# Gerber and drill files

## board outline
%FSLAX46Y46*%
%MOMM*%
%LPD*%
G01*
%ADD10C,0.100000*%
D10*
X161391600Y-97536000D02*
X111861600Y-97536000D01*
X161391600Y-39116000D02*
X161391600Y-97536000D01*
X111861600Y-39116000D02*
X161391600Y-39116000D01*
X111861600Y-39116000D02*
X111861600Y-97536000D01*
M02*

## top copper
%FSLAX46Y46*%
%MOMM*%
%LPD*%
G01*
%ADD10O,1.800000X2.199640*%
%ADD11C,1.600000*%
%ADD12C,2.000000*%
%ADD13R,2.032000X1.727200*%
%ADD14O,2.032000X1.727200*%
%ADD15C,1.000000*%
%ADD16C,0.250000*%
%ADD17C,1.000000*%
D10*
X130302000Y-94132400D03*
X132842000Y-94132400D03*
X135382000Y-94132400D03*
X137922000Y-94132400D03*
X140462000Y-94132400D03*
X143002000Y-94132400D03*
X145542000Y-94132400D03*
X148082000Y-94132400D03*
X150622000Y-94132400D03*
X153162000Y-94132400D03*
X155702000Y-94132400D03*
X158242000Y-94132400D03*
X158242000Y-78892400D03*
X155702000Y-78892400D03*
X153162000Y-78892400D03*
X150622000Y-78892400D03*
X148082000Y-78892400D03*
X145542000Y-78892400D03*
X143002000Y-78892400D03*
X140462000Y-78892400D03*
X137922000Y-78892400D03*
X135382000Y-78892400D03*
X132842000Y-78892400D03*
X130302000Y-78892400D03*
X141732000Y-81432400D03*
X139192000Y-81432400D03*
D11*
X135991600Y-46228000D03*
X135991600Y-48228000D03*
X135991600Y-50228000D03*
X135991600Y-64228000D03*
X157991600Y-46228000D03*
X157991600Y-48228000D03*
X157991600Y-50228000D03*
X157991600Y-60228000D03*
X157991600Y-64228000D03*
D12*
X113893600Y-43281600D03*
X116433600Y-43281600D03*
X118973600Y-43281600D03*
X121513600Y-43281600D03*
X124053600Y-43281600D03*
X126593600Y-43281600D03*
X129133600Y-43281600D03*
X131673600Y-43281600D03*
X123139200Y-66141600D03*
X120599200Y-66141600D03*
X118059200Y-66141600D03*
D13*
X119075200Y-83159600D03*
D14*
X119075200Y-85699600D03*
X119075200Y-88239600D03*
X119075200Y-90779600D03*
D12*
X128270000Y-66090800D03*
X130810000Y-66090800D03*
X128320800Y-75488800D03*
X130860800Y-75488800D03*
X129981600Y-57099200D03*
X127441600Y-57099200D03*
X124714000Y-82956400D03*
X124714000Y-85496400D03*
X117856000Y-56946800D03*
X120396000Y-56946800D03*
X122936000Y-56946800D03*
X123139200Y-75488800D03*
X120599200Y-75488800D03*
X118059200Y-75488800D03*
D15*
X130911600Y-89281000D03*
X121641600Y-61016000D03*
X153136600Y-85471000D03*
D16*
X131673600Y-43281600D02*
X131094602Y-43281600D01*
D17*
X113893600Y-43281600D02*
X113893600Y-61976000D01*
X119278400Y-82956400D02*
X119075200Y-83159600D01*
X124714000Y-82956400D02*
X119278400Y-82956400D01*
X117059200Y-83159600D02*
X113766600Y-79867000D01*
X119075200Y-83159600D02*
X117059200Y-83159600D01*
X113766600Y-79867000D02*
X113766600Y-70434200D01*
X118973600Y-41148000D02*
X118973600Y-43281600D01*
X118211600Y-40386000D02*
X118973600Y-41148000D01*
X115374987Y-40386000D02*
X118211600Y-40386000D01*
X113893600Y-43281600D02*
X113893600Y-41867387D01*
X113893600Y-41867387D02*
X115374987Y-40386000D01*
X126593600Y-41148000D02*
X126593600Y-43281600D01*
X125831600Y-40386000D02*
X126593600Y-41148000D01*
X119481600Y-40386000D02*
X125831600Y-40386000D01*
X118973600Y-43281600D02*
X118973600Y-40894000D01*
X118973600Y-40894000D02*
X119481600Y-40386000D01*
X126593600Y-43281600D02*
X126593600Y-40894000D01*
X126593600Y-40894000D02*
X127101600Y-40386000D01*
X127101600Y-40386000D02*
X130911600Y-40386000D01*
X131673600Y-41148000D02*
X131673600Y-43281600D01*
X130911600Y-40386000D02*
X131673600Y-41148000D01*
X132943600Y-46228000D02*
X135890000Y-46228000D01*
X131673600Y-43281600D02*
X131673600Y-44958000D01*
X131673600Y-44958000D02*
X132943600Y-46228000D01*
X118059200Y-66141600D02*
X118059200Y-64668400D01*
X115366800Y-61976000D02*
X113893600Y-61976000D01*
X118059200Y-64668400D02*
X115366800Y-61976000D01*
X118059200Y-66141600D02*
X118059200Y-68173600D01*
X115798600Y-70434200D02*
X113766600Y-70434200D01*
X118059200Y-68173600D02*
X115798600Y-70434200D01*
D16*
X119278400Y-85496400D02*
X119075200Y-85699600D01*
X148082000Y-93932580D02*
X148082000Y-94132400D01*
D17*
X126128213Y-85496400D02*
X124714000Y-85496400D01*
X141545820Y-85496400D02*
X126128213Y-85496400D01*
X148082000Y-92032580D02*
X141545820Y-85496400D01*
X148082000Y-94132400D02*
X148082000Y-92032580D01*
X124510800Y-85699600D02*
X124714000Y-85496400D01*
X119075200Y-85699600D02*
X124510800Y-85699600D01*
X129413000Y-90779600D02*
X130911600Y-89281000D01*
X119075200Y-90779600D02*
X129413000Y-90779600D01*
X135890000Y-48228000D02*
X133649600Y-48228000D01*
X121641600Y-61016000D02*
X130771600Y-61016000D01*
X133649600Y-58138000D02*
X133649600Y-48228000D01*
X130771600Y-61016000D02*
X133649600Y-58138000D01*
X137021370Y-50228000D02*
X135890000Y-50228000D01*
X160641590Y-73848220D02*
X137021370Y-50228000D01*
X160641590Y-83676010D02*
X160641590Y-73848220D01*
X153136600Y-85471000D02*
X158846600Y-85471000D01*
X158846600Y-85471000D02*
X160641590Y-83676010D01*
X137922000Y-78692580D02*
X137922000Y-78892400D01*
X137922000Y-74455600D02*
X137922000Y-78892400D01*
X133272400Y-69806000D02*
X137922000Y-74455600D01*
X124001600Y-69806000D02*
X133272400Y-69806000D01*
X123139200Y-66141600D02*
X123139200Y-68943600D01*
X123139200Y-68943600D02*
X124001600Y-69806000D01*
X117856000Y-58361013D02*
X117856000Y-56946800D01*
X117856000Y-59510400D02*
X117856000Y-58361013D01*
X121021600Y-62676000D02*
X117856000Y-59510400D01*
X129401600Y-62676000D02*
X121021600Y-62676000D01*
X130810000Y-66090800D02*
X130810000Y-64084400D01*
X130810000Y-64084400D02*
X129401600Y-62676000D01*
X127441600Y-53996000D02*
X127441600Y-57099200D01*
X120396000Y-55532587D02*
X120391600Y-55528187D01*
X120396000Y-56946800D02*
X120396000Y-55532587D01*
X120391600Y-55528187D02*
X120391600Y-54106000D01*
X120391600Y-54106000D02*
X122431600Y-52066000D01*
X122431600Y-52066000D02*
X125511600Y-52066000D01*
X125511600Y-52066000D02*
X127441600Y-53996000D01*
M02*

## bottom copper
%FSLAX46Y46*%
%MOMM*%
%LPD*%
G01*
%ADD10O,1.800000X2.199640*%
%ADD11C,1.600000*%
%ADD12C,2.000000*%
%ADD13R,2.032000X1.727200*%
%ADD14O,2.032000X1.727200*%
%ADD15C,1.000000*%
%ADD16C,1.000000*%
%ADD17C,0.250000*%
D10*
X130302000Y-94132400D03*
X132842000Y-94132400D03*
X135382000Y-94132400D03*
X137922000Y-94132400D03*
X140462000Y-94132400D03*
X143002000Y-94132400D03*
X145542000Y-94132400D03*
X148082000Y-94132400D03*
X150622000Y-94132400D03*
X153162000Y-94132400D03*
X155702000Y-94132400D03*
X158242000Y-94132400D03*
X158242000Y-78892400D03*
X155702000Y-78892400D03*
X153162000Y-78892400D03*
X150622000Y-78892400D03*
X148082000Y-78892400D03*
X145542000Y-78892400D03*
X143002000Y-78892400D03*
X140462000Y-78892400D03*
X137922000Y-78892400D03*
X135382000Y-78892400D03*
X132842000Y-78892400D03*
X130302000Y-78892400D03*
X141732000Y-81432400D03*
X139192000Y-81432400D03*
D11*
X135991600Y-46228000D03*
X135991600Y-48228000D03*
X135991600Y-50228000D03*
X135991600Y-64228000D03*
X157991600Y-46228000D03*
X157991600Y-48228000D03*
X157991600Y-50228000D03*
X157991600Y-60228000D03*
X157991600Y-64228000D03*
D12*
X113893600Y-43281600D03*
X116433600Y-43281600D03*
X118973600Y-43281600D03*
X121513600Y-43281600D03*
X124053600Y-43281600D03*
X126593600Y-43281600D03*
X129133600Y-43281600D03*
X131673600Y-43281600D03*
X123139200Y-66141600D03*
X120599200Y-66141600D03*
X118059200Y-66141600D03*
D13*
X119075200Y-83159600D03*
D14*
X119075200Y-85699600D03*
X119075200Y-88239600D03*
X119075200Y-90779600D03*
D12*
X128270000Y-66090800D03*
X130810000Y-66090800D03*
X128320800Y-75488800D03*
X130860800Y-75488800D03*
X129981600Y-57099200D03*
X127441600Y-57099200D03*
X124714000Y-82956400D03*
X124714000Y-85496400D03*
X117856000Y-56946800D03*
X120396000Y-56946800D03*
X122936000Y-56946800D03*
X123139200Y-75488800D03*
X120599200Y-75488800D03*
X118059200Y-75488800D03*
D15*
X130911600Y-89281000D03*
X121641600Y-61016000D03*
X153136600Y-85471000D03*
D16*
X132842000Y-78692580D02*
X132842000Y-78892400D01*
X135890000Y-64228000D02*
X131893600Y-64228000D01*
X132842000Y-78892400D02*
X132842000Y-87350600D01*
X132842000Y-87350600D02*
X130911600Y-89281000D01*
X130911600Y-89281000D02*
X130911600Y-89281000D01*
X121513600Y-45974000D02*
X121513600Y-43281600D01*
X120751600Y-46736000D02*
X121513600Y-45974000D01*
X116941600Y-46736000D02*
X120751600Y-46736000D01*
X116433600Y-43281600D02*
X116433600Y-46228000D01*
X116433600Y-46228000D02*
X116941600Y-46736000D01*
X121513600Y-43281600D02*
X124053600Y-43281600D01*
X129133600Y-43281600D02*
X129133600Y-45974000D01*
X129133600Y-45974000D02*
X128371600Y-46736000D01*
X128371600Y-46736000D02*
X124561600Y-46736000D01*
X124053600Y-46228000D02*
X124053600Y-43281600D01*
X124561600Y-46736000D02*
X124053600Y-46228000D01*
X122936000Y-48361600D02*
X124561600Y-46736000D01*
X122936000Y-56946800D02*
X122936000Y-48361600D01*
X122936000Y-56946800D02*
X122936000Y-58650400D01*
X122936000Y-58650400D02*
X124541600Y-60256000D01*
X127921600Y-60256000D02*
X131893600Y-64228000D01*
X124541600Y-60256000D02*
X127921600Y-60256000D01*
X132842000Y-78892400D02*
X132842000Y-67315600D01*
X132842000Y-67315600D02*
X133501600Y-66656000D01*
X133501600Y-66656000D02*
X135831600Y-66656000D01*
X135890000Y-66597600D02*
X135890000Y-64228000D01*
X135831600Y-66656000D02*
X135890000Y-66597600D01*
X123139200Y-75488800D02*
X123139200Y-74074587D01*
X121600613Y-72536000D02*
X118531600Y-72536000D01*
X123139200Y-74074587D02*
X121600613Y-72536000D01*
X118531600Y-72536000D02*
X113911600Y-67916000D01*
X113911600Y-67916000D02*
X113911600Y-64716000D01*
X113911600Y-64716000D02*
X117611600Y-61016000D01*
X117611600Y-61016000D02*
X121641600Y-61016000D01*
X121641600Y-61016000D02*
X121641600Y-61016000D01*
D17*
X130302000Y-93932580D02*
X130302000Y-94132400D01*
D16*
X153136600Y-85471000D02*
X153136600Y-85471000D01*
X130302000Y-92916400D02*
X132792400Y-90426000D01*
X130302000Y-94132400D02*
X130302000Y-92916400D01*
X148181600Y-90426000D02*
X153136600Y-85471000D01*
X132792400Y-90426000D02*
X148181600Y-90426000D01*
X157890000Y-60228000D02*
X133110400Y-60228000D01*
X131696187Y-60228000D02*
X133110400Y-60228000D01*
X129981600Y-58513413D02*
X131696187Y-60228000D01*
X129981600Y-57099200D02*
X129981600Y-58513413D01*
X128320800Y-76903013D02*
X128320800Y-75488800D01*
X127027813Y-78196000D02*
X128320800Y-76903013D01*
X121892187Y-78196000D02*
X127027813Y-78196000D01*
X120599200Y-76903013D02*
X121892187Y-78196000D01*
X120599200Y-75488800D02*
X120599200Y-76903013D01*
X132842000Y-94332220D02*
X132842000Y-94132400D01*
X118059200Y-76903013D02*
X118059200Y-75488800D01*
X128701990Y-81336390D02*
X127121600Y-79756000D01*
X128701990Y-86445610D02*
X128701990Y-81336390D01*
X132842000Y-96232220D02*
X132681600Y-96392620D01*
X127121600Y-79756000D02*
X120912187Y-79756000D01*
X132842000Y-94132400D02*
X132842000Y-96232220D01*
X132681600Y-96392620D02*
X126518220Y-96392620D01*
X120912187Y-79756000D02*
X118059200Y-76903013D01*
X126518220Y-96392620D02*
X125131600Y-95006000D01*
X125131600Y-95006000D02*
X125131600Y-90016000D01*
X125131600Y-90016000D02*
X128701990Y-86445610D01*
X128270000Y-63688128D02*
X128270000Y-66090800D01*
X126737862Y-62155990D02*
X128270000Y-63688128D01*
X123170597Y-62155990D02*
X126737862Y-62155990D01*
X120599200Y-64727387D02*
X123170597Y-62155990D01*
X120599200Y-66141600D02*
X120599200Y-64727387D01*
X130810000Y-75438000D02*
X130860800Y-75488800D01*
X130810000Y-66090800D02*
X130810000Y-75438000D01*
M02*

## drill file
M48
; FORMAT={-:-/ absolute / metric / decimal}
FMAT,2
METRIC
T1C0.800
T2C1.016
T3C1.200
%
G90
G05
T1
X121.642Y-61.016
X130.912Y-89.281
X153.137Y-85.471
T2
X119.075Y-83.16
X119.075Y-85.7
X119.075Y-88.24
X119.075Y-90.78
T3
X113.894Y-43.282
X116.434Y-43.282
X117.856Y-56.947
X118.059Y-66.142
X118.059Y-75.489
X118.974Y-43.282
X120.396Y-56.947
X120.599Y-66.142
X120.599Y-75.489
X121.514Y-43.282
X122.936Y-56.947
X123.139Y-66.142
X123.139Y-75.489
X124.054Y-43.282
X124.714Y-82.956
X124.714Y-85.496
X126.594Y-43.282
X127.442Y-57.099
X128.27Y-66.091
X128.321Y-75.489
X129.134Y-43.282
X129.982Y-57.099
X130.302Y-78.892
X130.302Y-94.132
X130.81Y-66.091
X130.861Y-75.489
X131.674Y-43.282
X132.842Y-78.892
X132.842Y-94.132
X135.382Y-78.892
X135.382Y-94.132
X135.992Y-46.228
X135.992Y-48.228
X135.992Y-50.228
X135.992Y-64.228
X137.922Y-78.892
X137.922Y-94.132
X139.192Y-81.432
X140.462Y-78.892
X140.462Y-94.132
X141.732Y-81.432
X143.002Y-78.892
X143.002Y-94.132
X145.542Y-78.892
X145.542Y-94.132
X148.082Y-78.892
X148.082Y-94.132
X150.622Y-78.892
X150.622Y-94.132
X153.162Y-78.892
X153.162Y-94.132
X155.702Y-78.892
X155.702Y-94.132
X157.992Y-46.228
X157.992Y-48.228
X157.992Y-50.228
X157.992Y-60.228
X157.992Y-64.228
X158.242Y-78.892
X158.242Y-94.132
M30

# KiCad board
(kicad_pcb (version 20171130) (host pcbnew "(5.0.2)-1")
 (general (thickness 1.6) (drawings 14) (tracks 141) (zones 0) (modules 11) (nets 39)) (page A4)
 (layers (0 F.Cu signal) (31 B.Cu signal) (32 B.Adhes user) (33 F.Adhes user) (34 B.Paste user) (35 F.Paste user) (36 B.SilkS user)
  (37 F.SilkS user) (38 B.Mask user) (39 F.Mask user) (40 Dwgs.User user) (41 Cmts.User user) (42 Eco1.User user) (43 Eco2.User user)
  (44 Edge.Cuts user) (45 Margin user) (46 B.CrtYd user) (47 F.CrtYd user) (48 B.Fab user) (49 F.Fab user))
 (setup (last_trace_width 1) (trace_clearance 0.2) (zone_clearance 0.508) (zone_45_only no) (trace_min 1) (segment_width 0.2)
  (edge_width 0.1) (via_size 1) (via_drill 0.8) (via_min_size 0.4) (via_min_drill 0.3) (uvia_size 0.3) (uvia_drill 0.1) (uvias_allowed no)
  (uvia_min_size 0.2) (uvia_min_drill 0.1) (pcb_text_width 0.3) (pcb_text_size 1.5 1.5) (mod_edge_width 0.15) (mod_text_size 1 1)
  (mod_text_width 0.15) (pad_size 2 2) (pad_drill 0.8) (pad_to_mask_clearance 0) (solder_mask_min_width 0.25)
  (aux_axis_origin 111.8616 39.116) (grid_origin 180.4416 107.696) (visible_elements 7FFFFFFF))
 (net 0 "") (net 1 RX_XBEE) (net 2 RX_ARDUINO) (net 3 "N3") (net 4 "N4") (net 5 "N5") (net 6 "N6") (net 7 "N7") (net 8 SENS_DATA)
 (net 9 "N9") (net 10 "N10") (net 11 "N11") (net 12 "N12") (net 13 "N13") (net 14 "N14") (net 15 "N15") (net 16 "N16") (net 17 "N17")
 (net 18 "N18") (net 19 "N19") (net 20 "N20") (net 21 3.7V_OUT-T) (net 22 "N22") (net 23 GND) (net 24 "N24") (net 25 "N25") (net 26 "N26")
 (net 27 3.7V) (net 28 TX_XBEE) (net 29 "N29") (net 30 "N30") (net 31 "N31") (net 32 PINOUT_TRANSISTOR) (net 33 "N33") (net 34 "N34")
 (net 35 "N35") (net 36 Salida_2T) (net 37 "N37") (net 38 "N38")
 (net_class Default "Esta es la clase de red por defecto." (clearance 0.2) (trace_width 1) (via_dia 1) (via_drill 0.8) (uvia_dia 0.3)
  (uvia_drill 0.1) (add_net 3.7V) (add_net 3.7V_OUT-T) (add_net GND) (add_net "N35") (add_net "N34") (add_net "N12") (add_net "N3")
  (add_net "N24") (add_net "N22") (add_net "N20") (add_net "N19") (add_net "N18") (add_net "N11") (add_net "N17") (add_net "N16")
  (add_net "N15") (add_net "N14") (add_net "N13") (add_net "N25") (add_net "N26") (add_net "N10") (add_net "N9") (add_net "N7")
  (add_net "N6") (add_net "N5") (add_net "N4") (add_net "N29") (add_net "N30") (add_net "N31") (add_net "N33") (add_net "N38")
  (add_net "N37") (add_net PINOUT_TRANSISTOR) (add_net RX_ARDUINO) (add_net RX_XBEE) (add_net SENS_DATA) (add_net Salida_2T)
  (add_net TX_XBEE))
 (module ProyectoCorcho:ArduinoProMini (layer F.Cu) (at 144.272 86.5124)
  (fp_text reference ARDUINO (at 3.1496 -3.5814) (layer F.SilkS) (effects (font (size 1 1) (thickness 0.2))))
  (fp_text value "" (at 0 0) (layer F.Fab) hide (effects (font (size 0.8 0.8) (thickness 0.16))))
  (pad 12 thru_hole oval (at -13.97 7.62) (size 1.8 2.19964) (drill 1.2) (layers *.Cu *.Mask) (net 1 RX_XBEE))
  (pad 11 thru_hole oval (at -11.43 7.62) (size 1.8 2.19964) (drill 1.2) (layers *.Cu *.Mask) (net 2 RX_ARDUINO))
  (pad 10 thru_hole oval (at -8.89 7.62) (size 1.8 2.19964) (drill 1.2) (layers *.Cu *.Mask) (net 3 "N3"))
  (pad 9 thru_hole oval (at -6.35 7.62) (size 1.8 2.19964) (drill 1.2) (layers *.Cu *.Mask) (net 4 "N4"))
  (pad 8 thru_hole oval (at -3.81 7.62) (size 1.8 2.19964) (drill 1.2) (layers *.Cu *.Mask) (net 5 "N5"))
  (pad 7 thru_hole oval (at -1.27 7.62) (size 1.8 2.19964) (drill 1.2) (layers *.Cu *.Mask) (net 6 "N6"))
  (pad 6 thru_hole oval (at 1.27 7.62) (size 1.8 2.19964) (drill 1.2) (layers *.Cu *.Mask) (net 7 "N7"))
  (pad 5 thru_hole oval (at 3.81 7.62) (size 1.8 2.19964) (drill 1.2) (layers *.Cu *.Mask) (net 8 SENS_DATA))
  (pad 4 thru_hole oval (at 6.35 7.62) (size 1.8 2.19964) (drill 1.2) (layers *.Cu *.Mask) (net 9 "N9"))
  (pad 3 thru_hole oval (at 8.89 7.62) (size 1.8 2.19964) (drill 1.2) (layers *.Cu *.Mask) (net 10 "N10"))
  (pad 2 thru_hole oval (at 11.43 7.62) (size 1.8 2.19964) (drill 1.2) (layers *.Cu *.Mask) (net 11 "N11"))
  (pad 1 thru_hole oval (at 13.97 7.62) (size 1.8 2.19964) (drill 1.2) (layers *.Cu *.Mask) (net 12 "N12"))
  (pad 24 thru_hole oval (at 13.97 -7.62) (size 1.8 2.19964) (drill 1.2) (layers *.Cu *.Mask) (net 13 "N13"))
  (pad 23 thru_hole oval (at 11.43 -7.62) (size 1.8 2.19964) (drill 1.2) (layers *.Cu *.Mask) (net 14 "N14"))
  (pad 22 thru_hole oval (at 8.89 -7.62) (size 1.8 2.19964) (drill 1.2) (layers *.Cu *.Mask) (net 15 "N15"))
  (pad 21 thru_hole oval (at 6.35 -7.62) (size 1.8 2.19964) (drill 1.2) (layers *.Cu *.Mask) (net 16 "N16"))
  (pad 20 thru_hole oval (at 3.81 -7.62) (size 1.8 2.19964) (drill 1.2) (layers *.Cu *.Mask) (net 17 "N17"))
  (pad 19 thru_hole oval (at 1.27 -7.62) (size 1.8 2.19964) (drill 1.2) (layers *.Cu *.Mask) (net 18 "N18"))
  (pad 18 thru_hole oval (at -1.27 -7.62) (size 1.8 2.19964) (drill 1.2) (layers *.Cu *.Mask) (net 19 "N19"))
  (pad 17 thru_hole oval (at -3.81 -7.62) (size 1.8 2.19964) (drill 1.2) (layers *.Cu *.Mask) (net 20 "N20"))
  (pad 16 thru_hole oval (at -6.35 -7.62) (size 1.8 2.19964) (drill 1.2) (layers *.Cu *.Mask) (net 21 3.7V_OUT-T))
  (pad 15 thru_hole oval (at -8.89 -7.62) (size 1.8 2.19964) (drill 1.2) (layers *.Cu *.Mask) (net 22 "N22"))
  (pad 14 thru_hole oval (at -11.43 -7.62) (size 1.8 2.19964) (drill 1.2) (layers *.Cu *.Mask) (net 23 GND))
  (pad 13 thru_hole oval (at -13.97 -7.62) (size 1.8 2.19964) (drill 1.2) (layers *.Cu *.Mask) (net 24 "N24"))
  (pad 25 thru_hole oval (at -2.54 -5.08) (size 1.8 2.19964) (drill 1.2) (layers *.Cu *.Mask) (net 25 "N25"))
  (pad 26 thru_hole oval (at -5.08 -5.08) (size 1.8 2.19964) (drill 1.2) (layers *.Cu *.Mask) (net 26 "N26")))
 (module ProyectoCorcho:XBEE (layer F.Cu) (at 134.7216 44.958)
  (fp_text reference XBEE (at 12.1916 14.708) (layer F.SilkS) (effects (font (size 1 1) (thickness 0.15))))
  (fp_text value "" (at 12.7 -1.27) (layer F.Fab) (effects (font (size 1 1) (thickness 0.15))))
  (pad 1 thru_hole circle (at 1.27 1.27) (size 1.6 1.6) (drill 1.2) (layers *.Cu *.Mask) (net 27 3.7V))
  (pad 2 thru_hole circle (at 1.27 3.27) (size 1.6 1.6) (drill 1.2) (layers *.Cu *.Mask) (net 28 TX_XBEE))
  (pad 3 thru_hole circle (at 1.27 5.27) (size 1.6 1.6) (drill 1.2) (layers *.Cu *.Mask) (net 1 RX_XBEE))
  (pad 4 thru_hole circle (at 1.27 19.27) (size 1.6 1.6) (drill 1.2) (layers *.Cu *.Mask) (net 23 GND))
  (pad 5 thru_hole circle (at 23.27 1.27) (size 1.6 1.6) (drill 1.2) (layers *.Cu *.Mask) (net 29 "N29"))
  (pad 6 thru_hole circle (at 23.27 3.27) (size 1.6 1.6) (drill 1.2) (layers *.Cu *.Mask) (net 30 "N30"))
  (pad 7 thru_hole circle (at 23.27 5.27) (size 1.6 1.6) (drill 1.2) (layers *.Cu *.Mask) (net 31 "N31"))
  (pad 8 thru_hole circle (at 23.27 15.27) (size 1.6 1.6) (drill 1.2) (layers *.Cu *.Mask) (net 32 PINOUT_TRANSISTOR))
  (pad 9 thru_hole circle (at 23.27 19.27) (size 1.6 1.6) (drill 1.2) (layers *.Cu *.Mask) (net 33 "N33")))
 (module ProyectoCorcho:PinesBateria (layer F.Cu) (at 112.6236 42.0116)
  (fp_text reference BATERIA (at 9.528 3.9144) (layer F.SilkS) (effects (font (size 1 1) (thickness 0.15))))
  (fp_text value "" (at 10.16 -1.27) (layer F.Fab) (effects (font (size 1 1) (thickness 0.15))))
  (pad 1 thru_hole circle (at 1.27 1.27) (size 2 2) (drill 1.2) (layers *.Cu *.Mask) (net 27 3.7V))
  (pad 2 thru_hole circle (at 3.81 1.27) (size 2 2) (drill 1.2) (layers *.Cu *.Mask) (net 23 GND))
  (pad 3 thru_hole circle (at 6.35 1.27) (size 2 2) (drill 1.2) (layers *.Cu *.Mask) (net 27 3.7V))
  (pad 4 thru_hole circle (at 8.89 1.27) (size 2 2) (drill 1.2) (layers *.Cu *.Mask) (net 23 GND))
  (pad 5 thru_hole circle (at 11.43 1.27) (size 2 2) (drill 1.2) (layers *.Cu *.Mask) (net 23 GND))
  (pad 6 thru_hole circle (at 13.97 1.27) (size 2 2) (drill 1.2) (layers *.Cu *.Mask) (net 27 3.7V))
  (pad 7 thru_hole circle (at 16.51 1.27) (size 2 2) (drill 1.2) (layers *.Cu *.Mask) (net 23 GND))
  (pad 8 thru_hole circle (at 19.05 1.27) (size 2 2) (drill 1.2) (layers *.Cu *.Mask) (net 27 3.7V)))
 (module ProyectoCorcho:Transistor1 (layer B.Cu) (at 120.5992 66.1416)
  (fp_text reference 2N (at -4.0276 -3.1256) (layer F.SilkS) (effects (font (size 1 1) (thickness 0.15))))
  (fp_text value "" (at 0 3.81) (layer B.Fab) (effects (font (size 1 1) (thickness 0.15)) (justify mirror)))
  (pad 3 thru_hole circle (at 2.54 0) (size 2 2) (drill 1.2) (layers *.Cu *.Mask) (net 21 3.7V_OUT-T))
  (pad 2 thru_hole circle (at 0 0) (size 2 2) (drill 1.2) (layers *.Cu *.Mask) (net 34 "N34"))
  (pad 1 thru_hole circle (at -2.54 0) (size 2 2) (drill 1.2) (layers *.Cu *.Mask) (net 27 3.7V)))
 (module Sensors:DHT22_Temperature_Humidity (layer F.Cu) (at 119.0752 86.9696 270)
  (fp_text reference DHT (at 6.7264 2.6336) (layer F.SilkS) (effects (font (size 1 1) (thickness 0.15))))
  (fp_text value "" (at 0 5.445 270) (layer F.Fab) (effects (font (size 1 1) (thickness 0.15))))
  (pad 1 thru_hole rect (at -3.81 0) (size 2.032 1.7272) (drill 1.016) (layers *.Cu *.Mask F.SilkS) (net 27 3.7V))
  (pad 2 thru_hole oval (at -1.27 0) (size 2.032 1.7272) (drill 1.016) (layers *.Cu *.Mask F.SilkS) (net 8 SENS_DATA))
  (pad 3 thru_hole oval (at 1.27 0) (size 2.032 1.7272) (drill 1.016) (layers *.Cu *.Mask F.SilkS) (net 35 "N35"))
  (pad 4 thru_hole oval (at 3.81 0) (size 2.032 1.7272) (drill 1.016) (layers *.Cu *.Mask F.SilkS) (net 23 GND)))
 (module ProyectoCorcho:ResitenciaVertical (layer F.Cu) (at 128.27 66.0908)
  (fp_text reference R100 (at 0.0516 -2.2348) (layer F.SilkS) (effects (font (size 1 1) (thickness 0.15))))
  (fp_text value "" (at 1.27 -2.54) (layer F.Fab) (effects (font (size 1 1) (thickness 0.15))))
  (pad 1 thru_hole circle (at 0 0) (size 2 2) (drill 1.2) (layers *.Cu *.Mask) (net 34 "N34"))
  (pad 2 thru_hole circle (at 2.54 0) (size 2 2) (drill 1.2) (layers *.Cu *.Mask) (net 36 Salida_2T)))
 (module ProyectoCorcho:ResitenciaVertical (layer F.Cu) (at 128.3208 75.4888)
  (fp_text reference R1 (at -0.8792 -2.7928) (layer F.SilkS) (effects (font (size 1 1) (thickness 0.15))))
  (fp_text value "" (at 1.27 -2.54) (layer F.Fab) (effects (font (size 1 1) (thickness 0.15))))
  (pad 1 thru_hole circle (at 0 0) (size 2 2) (drill 1.2) (layers *.Cu *.Mask) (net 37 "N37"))
  (pad 2 thru_hole circle (at 2.54 0) (size 2 2) (drill 1.2) (layers *.Cu *.Mask) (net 36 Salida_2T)))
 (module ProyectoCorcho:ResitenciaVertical (layer F.Cu) (at 127.4416 57.0992)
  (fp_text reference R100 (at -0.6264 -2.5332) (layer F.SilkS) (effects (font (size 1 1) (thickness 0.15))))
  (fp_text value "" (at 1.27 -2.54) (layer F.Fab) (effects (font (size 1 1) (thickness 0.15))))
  (pad 2 thru_hole circle (at 2.54 0) (size 2 2) (drill 1.2) (layers *.Cu *.Mask) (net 32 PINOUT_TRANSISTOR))
  (pad 1 thru_hole circle (at 0 0) (size 2 2) (drill 1.2) (layers *.Cu *.Mask) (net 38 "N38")))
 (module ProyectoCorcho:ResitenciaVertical (layer F.Cu) (at 124.714 82.9564 270)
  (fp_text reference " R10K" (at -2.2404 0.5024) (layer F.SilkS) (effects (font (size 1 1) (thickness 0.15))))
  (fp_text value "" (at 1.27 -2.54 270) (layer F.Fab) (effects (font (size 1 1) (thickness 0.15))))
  (pad 1 thru_hole circle (at 0 0 270) (size 2 2) (drill 1.2) (layers *.Cu *.Mask) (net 27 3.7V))
  (pad 2 thru_hole circle (at 2.54 0 270) (size 2 2) (drill 1.2) (layers *.Cu *.Mask) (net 8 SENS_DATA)))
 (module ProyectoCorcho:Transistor (layer F.Cu) (at 120.396 56.9468)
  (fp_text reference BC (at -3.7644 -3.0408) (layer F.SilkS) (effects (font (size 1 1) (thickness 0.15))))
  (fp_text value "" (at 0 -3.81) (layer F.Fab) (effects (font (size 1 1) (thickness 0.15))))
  (pad 1 thru_hole circle (at -2.54 0) (size 2 2) (drill 1.2) (layers *.Cu *.Mask) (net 36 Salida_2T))
  (pad 2 thru_hole circle (at 0 0) (size 2 2) (drill 1.2) (layers *.Cu *.Mask) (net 38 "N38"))
  (pad 3 thru_hole circle (at 2.54 0) (size 2 2) (drill 1.2) (layers *.Cu *.Mask) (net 23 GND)))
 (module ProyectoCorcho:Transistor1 (layer B.Cu) (at 120.5992 75.4888 180)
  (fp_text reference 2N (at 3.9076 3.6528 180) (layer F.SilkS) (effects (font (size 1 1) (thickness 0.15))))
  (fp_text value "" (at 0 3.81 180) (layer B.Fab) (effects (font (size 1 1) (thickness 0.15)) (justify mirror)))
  (pad 1 thru_hole circle (at -2.54 0 180) (size 2 2) (drill 1.2) (layers *.Cu *.Mask) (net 28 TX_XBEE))
  (pad 2 thru_hole circle (at 0 0 180) (size 2 2) (drill 1.2) (layers *.Cu *.Mask) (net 37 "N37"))
  (pad 3 thru_hole circle (at 2.54 0 180) (size 2 2) (drill 1.2) (layers *.Cu *.Mask) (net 2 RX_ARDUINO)))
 (gr_line (start 161.3916 97.536) (end 111.8616 97.536) (layer Edge.Cuts) (width 0.1))
 (gr_line (start 161.3916 39.116) (end 161.3916 97.536) (layer Edge.Cuts) (width 0.1))
 (gr_line (start 111.8616 39.116) (end 161.3916 39.116) (layer Edge.Cuts) (width 0.1))
 (gr_line (start 111.8616 39.116) (end 111.8616 97.536) (layer Edge.Cuts) (width 0.1))
 (segment (start 131.6736 43.2816) (end 131.094602 43.2816) (width 0.25) (layer F.Cu) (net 27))
 (segment (start 113.8936 43.2816) (end 113.8936 61.976) (width 1) (layer F.Cu) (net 27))
 (segment (start 119.2784 82.9564) (end 119.0752 83.1596) (width 1) (layer F.Cu) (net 27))
 (segment (start 124.714 82.9564) (end 119.2784 82.9564) (width 1) (layer F.Cu) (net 27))
 (segment (start 117.0592 83.1596) (end 113.7666 79.867) (width 1) (layer F.Cu) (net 27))
 (segment (start 119.0752 83.1596) (end 117.0592 83.1596) (width 1) (layer F.Cu) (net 27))
 (segment (start 113.7666 79.867) (end 113.7666 70.4342) (width 1) (layer F.Cu) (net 27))
 (segment (start 118.9736 41.148) (end 118.9736 43.2816) (width 1) (layer F.Cu) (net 27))
 (segment (start 118.2116 40.386) (end 118.9736 41.148) (width 1) (layer F.Cu) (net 27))
 (segment (start 115.374987 40.386) (end 118.2116 40.386) (width 1) (layer F.Cu) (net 27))
 (segment (start 113.8936 43.2816) (end 113.8936 41.867387) (width 1) (layer F.Cu) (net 27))
 (segment (start 113.8936 41.867387) (end 115.374987 40.386) (width 1) (layer F.Cu) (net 27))
 (segment (start 126.5936 41.148) (end 126.5936 43.2816) (width 1) (layer F.Cu) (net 27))
 (segment (start 125.8316 40.386) (end 126.5936 41.148) (width 1) (layer F.Cu) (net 27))
 (segment (start 119.4816 40.386) (end 125.8316 40.386) (width 1) (layer F.Cu) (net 27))
 (segment (start 118.9736 43.2816) (end 118.9736 40.894) (width 1) (layer F.Cu) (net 27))
 (segment (start 118.9736 40.894) (end 119.4816 40.386) (width 1) (layer F.Cu) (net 27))
 (segment (start 126.5936 43.2816) (end 126.5936 40.894) (width 1) (layer F.Cu) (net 27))
 (segment (start 126.5936 40.894) (end 127.1016 40.386) (width 1) (layer F.Cu) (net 27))
 (segment (start 127.1016 40.386) (end 130.9116 40.386) (width 1) (layer F.Cu) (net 27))
 (segment (start 131.6736 41.148) (end 131.6736 43.2816) (width 1) (layer F.Cu) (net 27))
 (segment (start 130.9116 40.386) (end 131.6736 41.148) (width 1) (layer F.Cu) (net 27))
 (segment (start 132.9436 46.228) (end 135.89 46.228) (width 1) (layer F.Cu) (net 27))
 (segment (start 131.6736 43.2816) (end 131.6736 44.958) (width 1) (layer F.Cu) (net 27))
 (segment (start 131.6736 44.958) (end 132.9436 46.228) (width 1) (layer F.Cu) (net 27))
 (segment (start 118.0592 66.1416) (end 118.0592 64.6684) (width 1) (layer F.Cu) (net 27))
 (segment (start 115.3668 61.976) (end 113.8936 61.976) (width 1) (layer F.Cu) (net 27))
 (segment (start 118.0592 64.6684) (end 115.3668 61.976) (width 1) (layer F.Cu) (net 27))
 (segment (start 118.0592 66.1416) (end 118.0592 68.1736) (width 1) (layer F.Cu) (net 27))
 (segment (start 115.7986 70.4342) (end 113.7666 70.4342) (width 1) (layer F.Cu) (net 27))
 (segment (start 118.0592 68.1736) (end 115.7986 70.4342) (width 1) (layer F.Cu) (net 27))
 (segment (start 119.2784 85.4964) (end 119.0752 85.6996) (width 0.25) (layer F.Cu) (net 8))
 (segment (start 148.082 93.93258) (end 148.082 94.1324) (width 0.25) (layer F.Cu) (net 8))
 (segment (start 126.128213 85.4964) (end 124.714 85.4964) (width 1) (layer F.Cu) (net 8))
 (segment (start 141.54582 85.4964) (end 126.128213 85.4964) (width 1) (layer F.Cu) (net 8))
 (segment (start 148.082 92.03258) (end 141.54582 85.4964) (width 1) (layer F.Cu) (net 8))
 (segment (start 148.082 94.1324) (end 148.082 92.03258) (width 1) (layer F.Cu) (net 8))
 (segment (start 124.5108 85.6996) (end 124.714 85.4964) (width 1) (layer F.Cu) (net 8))
 (segment (start 119.0752 85.6996) (end 124.5108 85.6996) (width 1) (layer F.Cu) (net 8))
 (segment (start 132.842 78.69258) (end 132.842 78.8924) (width 1) (layer B.Cu) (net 23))
 (segment (start 135.89 64.228) (end 131.8936 64.228) (width 1) (layer B.Cu) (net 23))
 (segment (start 132.842 78.8924) (end 132.842 87.3506) (width 1) (layer B.Cu) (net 23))
 (segment (start 132.842 87.3506) (end 130.9116 89.281) (width 1) (layer B.Cu) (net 23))
 (segment (start 130.9116 89.281) (end 130.9116 89.281) (width 1) (layer B.Cu) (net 23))
 (via (at 130.9116 89.281) (size 1) (drill 0.8) (layers F.Cu B.Cu) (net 23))
 (segment (start 129.413 90.7796) (end 130.9116 89.281) (width 1) (layer F.Cu) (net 23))
 (segment (start 119.0752 90.7796) (end 129.413 90.7796) (width 1) (layer F.Cu) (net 23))
 (segment (start 121.5136 45.974) (end 121.5136 43.2816) (width 1) (layer B.Cu) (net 23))
 (segment (start 120.7516 46.736) (end 121.5136 45.974) (width 1) (layer B.Cu) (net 23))
 (segment (start 116.9416 46.736) (end 120.7516 46.736) (width 1) (layer B.Cu) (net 23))
 (segment (start 116.4336 43.2816) (end 116.4336 46.228) (width 1) (layer B.Cu) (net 23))
 (segment (start 116.4336 46.228) (end 116.9416 46.736) (width 1) (layer B.Cu) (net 23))
 (segment (start 121.5136 43.2816) (end 124.0536 43.2816) (width 1) (layer B.Cu) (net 23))
 (segment (start 129.1336 43.2816) (end 129.1336 45.974) (width 1) (layer B.Cu) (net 23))
 (segment (start 129.1336 45.974) (end 128.3716 46.736) (width 1) (layer B.Cu) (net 23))
 (segment (start 128.3716 46.736) (end 124.5616 46.736) (width 1) (layer B.Cu) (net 23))
 (segment (start 124.0536 46.228) (end 124.0536 43.2816) (width 1) (layer B.Cu) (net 23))
 (segment (start 124.5616 46.736) (end 124.0536 46.228) (width 1) (layer B.Cu) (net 23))
 (segment (start 122.936 48.3616) (end 124.5616 46.736) (width 1) (layer B.Cu) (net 23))
 (segment (start 122.936 56.9468) (end 122.936 48.3616) (width 1) (layer B.Cu) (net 23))
 (segment (start 122.936 56.9468) (end 122.936 58.6504) (width 1) (layer B.Cu) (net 23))
 (segment (start 122.936 58.6504) (end 124.5416 60.256) (width 1) (layer B.Cu) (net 23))
 (segment (start 127.9216 60.256) (end 131.8936 64.228) (width 1) (layer B.Cu) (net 23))
 (segment (start 124.5416 60.256) (end 127.9216 60.256) (width 1) (layer B.Cu) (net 23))
 (segment (start 132.842 78.8924) (end 132.842 67.3156) (width 1) (layer B.Cu) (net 23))
 (segment (start 132.842 67.3156) (end 133.5016 66.656) (width 1) (layer B.Cu) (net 23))
 (segment (start 133.5016 66.656) (end 135.8316 66.656) (width 1) (layer B.Cu) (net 23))
 (segment (start 135.89 66.5976) (end 135.89 64.228) (width 1) (layer B.Cu) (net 23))
 (segment (start 135.8316 66.656) (end 135.89 66.5976) (width 1) (layer B.Cu) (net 23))
 (segment (start 123.1392 75.4888) (end 123.1392 74.074587) (width 1) (layer B.Cu) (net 28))
 (segment (start 135.89 48.228) (end 133.6496 48.228) (width 1) (layer F.Cu) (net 28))
 (segment (start 121.600613 72.536) (end 118.5316 72.536) (width 1) (layer B.Cu) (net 28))
 (segment (start 123.1392 74.074587) (end 121.600613 72.536) (width 1) (layer B.Cu) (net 28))
 (segment (start 118.5316 72.536) (end 113.9116 67.916) (width 1) (layer B.Cu) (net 28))
 (segment (start 113.9116 67.916) (end 113.9116 64.716) (width 1) (layer B.Cu) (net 28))
 (segment (start 113.9116 64.716) (end 117.6116 61.016) (width 1) (layer B.Cu) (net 28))
 (segment (start 117.6116 61.016) (end 121.6416 61.016) (width 1) (layer B.Cu) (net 28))
 (segment (start 121.6416 61.016) (end 121.6416 61.016) (width 1) (layer B.Cu) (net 28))
 (via (at 121.6416 61.016) (size 1) (drill 0.8) (layers F.Cu B.Cu) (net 28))
 (segment (start 121.6416 61.016) (end 130.7716 61.016) (width 1) (layer F.Cu) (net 28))
 (segment (start 133.6496 58.138) (end 133.6496 48.228) (width 1) (layer F.Cu) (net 28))
 (segment (start 130.7716 61.016) (end 133.6496 58.138) (width 1) (layer F.Cu) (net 28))
 (segment (start 130.302 93.93258) (end 130.302 94.1324) (width 0.25) (layer B.Cu) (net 1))
 (segment (start 153.1366 85.471) (end 153.1366 85.471) (width 1) (layer B.Cu) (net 1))
 (via (at 153.1366 85.471) (size 1) (drill 0.8) (layers F.Cu B.Cu) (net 1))
 (segment (start 130.302 92.9164) (end 132.7924 90.426) (width 1) (layer B.Cu) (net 1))
 (segment (start 130.302 94.1324) (end 130.302 92.9164) (width 1) (layer B.Cu) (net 1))
 (segment (start 148.1816 90.426) (end 153.1366 85.471) (width 1) (layer B.Cu) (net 1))
 (segment (start 132.7924 90.426) (end 148.1816 90.426) (width 1) (layer B.Cu) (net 1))
 (segment (start 137.02137 50.228) (end 135.89 50.228) (width 1) (layer F.Cu) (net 1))
 (segment (start 160.64159 73.84822) (end 137.02137 50.228) (width 1) (layer F.Cu) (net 1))
 (segment (start 160.64159 83.67601) (end 160.64159 73.84822) (width 1) (layer F.Cu) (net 1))
 (segment (start 153.1366 85.471) (end 158.8466 85.471) (width 1) (layer F.Cu) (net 1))
 (segment (start 158.8466 85.471) (end 160.64159 83.67601) (width 1) (layer F.Cu) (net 1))
 (segment (start 157.89 60.228) (end 133.1104 60.228) (width 1) (layer B.Cu) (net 32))
 (segment (start 131.696187 60.228) (end 133.1104 60.228) (width 1) (layer B.Cu) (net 32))
 (segment (start 129.9816 58.513413) (end 131.696187 60.228) (width 1) (layer B.Cu) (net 32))
 (segment (start 129.9816 57.0992) (end 129.9816 58.513413) (width 1) (layer B.Cu) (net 32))
 (segment (start 128.3208 76.903013) (end 128.3208 75.4888) (width 1) (layer B.Cu) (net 37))
 (segment (start 127.027813 78.196) (end 128.3208 76.903013) (width 1) (layer B.Cu) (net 37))
 (segment (start 121.892187 78.196) (end 127.027813 78.196) (width 1) (layer B.Cu) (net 37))
 (segment (start 120.5992 76.903013) (end 121.892187 78.196) (width 1) (layer B.Cu) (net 37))
 (segment (start 120.5992 75.4888) (end 120.5992 76.903013) (width 1) (layer B.Cu) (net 37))
 (segment (start 132.842 94.33222) (end 132.842 94.1324) (width 1) (layer B.Cu) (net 2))
 (segment (start 118.0592 76.903013) (end 118.0592 75.4888) (width 1) (layer B.Cu) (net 2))
 (segment (start 128.70199 81.33639) (end 127.1216 79.756) (width 1) (layer B.Cu) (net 2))
 (segment (start 128.70199 86.44561) (end 128.70199 81.33639) (width 1) (layer B.Cu) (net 2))
 (segment (start 132.842 96.23222) (end 132.6816 96.39262) (width 1) (layer B.Cu) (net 2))
 (segment (start 127.1216 79.756) (end 120.912187 79.756) (width 1) (layer B.Cu) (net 2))
 (segment (start 132.842 94.1324) (end 132.842 96.23222) (width 1) (layer B.Cu) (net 2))
 (segment (start 132.6816 96.39262) (end 126.51822 96.39262) (width 1) (layer B.Cu) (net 2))
 (segment (start 120.912187 79.756) (end 118.0592 76.903013) (width 1) (layer B.Cu) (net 2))
 (segment (start 126.51822 96.39262) (end 125.1316 95.006) (width 1) (layer B.Cu) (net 2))
 (segment (start 125.1316 95.006) (end 125.1316 90.016) (width 1) (layer B.Cu) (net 2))
 (segment (start 125.1316 90.016) (end 128.70199 86.44561) (width 1) (layer B.Cu) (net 2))
 (segment (start 137.922 78.69258) (end 137.922 78.8924) (width 1) (layer F.Cu) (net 21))
 (segment (start 137.922 74.4556) (end 137.922 78.8924) (width 1) (layer F.Cu) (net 21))
 (segment (start 133.2724 69.806) (end 137.922 74.4556) (width 1) (layer F.Cu) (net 21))
 (segment (start 124.0016 69.806) (end 133.2724 69.806) (width 1) (layer F.Cu) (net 21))
 (segment (start 123.1392 66.1416) (end 123.1392 68.9436) (width 1) (layer F.Cu) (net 21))
 (segment (start 123.1392 68.9436) (end 124.0016 69.806) (width 1) (layer F.Cu) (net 21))
 (segment (start 128.27 63.688128) (end 128.27 66.0908) (width 1) (layer B.Cu) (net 34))
 (segment (start 126.737862 62.15599) (end 128.27 63.688128) (width 1) (layer B.Cu) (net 34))
 (segment (start 123.170597 62.15599) (end 126.737862 62.15599) (width 1) (layer B.Cu) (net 34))
 (segment (start 120.5992 64.727387) (end 123.170597 62.15599) (width 1) (layer B.Cu) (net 34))
 (segment (start 120.5992 66.1416) (end 120.5992 64.727387) (width 1) (layer B.Cu) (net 34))
 (segment (start 130.81 75.438) (end 130.8608 75.4888) (width 1) (layer B.Cu) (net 36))
 (segment (start 130.81 66.0908) (end 130.81 75.438) (width 1) (layer B.Cu) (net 36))
 (segment (start 117.856 58.361013) (end 117.856 56.9468) (width 1) (layer F.Cu) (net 36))
 (segment (start 117.856 59.5104) (end 117.856 58.361013) (width 1) (layer F.Cu) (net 36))
 (segment (start 121.0216 62.676) (end 117.856 59.5104) (width 1) (layer F.Cu) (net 36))
 (segment (start 129.4016 62.676) (end 121.0216 62.676) (width 1) (layer F.Cu) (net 36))
 (segment (start 130.81 66.0908) (end 130.81 64.0844) (width 1) (layer F.Cu) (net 36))
 (segment (start 130.81 64.0844) (end 129.4016 62.676) (width 1) (layer F.Cu) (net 36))
 (segment (start 127.4416 53.996) (end 127.4416 57.0992) (width 1) (layer F.Cu) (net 38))
 (segment (start 120.396 55.532587) (end 120.3916 55.528187) (width 1) (layer F.Cu) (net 38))
 (segment (start 120.396 56.9468) (end 120.396 55.532587) (width 1) (layer F.Cu) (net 38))
 (segment (start 120.3916 55.528187) (end 120.3916 54.106) (width 1) (layer F.Cu) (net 38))
 (segment (start 120.3916 54.106) (end 122.4316 52.066) (width 1) (layer F.Cu) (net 38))
 (segment (start 122.4316 52.066) (end 125.5116 52.066) (width 1) (layer F.Cu) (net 38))
 (segment (start 125.5116 52.066) (end 127.4416 53.996) (width 1) (layer F.Cu) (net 38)))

